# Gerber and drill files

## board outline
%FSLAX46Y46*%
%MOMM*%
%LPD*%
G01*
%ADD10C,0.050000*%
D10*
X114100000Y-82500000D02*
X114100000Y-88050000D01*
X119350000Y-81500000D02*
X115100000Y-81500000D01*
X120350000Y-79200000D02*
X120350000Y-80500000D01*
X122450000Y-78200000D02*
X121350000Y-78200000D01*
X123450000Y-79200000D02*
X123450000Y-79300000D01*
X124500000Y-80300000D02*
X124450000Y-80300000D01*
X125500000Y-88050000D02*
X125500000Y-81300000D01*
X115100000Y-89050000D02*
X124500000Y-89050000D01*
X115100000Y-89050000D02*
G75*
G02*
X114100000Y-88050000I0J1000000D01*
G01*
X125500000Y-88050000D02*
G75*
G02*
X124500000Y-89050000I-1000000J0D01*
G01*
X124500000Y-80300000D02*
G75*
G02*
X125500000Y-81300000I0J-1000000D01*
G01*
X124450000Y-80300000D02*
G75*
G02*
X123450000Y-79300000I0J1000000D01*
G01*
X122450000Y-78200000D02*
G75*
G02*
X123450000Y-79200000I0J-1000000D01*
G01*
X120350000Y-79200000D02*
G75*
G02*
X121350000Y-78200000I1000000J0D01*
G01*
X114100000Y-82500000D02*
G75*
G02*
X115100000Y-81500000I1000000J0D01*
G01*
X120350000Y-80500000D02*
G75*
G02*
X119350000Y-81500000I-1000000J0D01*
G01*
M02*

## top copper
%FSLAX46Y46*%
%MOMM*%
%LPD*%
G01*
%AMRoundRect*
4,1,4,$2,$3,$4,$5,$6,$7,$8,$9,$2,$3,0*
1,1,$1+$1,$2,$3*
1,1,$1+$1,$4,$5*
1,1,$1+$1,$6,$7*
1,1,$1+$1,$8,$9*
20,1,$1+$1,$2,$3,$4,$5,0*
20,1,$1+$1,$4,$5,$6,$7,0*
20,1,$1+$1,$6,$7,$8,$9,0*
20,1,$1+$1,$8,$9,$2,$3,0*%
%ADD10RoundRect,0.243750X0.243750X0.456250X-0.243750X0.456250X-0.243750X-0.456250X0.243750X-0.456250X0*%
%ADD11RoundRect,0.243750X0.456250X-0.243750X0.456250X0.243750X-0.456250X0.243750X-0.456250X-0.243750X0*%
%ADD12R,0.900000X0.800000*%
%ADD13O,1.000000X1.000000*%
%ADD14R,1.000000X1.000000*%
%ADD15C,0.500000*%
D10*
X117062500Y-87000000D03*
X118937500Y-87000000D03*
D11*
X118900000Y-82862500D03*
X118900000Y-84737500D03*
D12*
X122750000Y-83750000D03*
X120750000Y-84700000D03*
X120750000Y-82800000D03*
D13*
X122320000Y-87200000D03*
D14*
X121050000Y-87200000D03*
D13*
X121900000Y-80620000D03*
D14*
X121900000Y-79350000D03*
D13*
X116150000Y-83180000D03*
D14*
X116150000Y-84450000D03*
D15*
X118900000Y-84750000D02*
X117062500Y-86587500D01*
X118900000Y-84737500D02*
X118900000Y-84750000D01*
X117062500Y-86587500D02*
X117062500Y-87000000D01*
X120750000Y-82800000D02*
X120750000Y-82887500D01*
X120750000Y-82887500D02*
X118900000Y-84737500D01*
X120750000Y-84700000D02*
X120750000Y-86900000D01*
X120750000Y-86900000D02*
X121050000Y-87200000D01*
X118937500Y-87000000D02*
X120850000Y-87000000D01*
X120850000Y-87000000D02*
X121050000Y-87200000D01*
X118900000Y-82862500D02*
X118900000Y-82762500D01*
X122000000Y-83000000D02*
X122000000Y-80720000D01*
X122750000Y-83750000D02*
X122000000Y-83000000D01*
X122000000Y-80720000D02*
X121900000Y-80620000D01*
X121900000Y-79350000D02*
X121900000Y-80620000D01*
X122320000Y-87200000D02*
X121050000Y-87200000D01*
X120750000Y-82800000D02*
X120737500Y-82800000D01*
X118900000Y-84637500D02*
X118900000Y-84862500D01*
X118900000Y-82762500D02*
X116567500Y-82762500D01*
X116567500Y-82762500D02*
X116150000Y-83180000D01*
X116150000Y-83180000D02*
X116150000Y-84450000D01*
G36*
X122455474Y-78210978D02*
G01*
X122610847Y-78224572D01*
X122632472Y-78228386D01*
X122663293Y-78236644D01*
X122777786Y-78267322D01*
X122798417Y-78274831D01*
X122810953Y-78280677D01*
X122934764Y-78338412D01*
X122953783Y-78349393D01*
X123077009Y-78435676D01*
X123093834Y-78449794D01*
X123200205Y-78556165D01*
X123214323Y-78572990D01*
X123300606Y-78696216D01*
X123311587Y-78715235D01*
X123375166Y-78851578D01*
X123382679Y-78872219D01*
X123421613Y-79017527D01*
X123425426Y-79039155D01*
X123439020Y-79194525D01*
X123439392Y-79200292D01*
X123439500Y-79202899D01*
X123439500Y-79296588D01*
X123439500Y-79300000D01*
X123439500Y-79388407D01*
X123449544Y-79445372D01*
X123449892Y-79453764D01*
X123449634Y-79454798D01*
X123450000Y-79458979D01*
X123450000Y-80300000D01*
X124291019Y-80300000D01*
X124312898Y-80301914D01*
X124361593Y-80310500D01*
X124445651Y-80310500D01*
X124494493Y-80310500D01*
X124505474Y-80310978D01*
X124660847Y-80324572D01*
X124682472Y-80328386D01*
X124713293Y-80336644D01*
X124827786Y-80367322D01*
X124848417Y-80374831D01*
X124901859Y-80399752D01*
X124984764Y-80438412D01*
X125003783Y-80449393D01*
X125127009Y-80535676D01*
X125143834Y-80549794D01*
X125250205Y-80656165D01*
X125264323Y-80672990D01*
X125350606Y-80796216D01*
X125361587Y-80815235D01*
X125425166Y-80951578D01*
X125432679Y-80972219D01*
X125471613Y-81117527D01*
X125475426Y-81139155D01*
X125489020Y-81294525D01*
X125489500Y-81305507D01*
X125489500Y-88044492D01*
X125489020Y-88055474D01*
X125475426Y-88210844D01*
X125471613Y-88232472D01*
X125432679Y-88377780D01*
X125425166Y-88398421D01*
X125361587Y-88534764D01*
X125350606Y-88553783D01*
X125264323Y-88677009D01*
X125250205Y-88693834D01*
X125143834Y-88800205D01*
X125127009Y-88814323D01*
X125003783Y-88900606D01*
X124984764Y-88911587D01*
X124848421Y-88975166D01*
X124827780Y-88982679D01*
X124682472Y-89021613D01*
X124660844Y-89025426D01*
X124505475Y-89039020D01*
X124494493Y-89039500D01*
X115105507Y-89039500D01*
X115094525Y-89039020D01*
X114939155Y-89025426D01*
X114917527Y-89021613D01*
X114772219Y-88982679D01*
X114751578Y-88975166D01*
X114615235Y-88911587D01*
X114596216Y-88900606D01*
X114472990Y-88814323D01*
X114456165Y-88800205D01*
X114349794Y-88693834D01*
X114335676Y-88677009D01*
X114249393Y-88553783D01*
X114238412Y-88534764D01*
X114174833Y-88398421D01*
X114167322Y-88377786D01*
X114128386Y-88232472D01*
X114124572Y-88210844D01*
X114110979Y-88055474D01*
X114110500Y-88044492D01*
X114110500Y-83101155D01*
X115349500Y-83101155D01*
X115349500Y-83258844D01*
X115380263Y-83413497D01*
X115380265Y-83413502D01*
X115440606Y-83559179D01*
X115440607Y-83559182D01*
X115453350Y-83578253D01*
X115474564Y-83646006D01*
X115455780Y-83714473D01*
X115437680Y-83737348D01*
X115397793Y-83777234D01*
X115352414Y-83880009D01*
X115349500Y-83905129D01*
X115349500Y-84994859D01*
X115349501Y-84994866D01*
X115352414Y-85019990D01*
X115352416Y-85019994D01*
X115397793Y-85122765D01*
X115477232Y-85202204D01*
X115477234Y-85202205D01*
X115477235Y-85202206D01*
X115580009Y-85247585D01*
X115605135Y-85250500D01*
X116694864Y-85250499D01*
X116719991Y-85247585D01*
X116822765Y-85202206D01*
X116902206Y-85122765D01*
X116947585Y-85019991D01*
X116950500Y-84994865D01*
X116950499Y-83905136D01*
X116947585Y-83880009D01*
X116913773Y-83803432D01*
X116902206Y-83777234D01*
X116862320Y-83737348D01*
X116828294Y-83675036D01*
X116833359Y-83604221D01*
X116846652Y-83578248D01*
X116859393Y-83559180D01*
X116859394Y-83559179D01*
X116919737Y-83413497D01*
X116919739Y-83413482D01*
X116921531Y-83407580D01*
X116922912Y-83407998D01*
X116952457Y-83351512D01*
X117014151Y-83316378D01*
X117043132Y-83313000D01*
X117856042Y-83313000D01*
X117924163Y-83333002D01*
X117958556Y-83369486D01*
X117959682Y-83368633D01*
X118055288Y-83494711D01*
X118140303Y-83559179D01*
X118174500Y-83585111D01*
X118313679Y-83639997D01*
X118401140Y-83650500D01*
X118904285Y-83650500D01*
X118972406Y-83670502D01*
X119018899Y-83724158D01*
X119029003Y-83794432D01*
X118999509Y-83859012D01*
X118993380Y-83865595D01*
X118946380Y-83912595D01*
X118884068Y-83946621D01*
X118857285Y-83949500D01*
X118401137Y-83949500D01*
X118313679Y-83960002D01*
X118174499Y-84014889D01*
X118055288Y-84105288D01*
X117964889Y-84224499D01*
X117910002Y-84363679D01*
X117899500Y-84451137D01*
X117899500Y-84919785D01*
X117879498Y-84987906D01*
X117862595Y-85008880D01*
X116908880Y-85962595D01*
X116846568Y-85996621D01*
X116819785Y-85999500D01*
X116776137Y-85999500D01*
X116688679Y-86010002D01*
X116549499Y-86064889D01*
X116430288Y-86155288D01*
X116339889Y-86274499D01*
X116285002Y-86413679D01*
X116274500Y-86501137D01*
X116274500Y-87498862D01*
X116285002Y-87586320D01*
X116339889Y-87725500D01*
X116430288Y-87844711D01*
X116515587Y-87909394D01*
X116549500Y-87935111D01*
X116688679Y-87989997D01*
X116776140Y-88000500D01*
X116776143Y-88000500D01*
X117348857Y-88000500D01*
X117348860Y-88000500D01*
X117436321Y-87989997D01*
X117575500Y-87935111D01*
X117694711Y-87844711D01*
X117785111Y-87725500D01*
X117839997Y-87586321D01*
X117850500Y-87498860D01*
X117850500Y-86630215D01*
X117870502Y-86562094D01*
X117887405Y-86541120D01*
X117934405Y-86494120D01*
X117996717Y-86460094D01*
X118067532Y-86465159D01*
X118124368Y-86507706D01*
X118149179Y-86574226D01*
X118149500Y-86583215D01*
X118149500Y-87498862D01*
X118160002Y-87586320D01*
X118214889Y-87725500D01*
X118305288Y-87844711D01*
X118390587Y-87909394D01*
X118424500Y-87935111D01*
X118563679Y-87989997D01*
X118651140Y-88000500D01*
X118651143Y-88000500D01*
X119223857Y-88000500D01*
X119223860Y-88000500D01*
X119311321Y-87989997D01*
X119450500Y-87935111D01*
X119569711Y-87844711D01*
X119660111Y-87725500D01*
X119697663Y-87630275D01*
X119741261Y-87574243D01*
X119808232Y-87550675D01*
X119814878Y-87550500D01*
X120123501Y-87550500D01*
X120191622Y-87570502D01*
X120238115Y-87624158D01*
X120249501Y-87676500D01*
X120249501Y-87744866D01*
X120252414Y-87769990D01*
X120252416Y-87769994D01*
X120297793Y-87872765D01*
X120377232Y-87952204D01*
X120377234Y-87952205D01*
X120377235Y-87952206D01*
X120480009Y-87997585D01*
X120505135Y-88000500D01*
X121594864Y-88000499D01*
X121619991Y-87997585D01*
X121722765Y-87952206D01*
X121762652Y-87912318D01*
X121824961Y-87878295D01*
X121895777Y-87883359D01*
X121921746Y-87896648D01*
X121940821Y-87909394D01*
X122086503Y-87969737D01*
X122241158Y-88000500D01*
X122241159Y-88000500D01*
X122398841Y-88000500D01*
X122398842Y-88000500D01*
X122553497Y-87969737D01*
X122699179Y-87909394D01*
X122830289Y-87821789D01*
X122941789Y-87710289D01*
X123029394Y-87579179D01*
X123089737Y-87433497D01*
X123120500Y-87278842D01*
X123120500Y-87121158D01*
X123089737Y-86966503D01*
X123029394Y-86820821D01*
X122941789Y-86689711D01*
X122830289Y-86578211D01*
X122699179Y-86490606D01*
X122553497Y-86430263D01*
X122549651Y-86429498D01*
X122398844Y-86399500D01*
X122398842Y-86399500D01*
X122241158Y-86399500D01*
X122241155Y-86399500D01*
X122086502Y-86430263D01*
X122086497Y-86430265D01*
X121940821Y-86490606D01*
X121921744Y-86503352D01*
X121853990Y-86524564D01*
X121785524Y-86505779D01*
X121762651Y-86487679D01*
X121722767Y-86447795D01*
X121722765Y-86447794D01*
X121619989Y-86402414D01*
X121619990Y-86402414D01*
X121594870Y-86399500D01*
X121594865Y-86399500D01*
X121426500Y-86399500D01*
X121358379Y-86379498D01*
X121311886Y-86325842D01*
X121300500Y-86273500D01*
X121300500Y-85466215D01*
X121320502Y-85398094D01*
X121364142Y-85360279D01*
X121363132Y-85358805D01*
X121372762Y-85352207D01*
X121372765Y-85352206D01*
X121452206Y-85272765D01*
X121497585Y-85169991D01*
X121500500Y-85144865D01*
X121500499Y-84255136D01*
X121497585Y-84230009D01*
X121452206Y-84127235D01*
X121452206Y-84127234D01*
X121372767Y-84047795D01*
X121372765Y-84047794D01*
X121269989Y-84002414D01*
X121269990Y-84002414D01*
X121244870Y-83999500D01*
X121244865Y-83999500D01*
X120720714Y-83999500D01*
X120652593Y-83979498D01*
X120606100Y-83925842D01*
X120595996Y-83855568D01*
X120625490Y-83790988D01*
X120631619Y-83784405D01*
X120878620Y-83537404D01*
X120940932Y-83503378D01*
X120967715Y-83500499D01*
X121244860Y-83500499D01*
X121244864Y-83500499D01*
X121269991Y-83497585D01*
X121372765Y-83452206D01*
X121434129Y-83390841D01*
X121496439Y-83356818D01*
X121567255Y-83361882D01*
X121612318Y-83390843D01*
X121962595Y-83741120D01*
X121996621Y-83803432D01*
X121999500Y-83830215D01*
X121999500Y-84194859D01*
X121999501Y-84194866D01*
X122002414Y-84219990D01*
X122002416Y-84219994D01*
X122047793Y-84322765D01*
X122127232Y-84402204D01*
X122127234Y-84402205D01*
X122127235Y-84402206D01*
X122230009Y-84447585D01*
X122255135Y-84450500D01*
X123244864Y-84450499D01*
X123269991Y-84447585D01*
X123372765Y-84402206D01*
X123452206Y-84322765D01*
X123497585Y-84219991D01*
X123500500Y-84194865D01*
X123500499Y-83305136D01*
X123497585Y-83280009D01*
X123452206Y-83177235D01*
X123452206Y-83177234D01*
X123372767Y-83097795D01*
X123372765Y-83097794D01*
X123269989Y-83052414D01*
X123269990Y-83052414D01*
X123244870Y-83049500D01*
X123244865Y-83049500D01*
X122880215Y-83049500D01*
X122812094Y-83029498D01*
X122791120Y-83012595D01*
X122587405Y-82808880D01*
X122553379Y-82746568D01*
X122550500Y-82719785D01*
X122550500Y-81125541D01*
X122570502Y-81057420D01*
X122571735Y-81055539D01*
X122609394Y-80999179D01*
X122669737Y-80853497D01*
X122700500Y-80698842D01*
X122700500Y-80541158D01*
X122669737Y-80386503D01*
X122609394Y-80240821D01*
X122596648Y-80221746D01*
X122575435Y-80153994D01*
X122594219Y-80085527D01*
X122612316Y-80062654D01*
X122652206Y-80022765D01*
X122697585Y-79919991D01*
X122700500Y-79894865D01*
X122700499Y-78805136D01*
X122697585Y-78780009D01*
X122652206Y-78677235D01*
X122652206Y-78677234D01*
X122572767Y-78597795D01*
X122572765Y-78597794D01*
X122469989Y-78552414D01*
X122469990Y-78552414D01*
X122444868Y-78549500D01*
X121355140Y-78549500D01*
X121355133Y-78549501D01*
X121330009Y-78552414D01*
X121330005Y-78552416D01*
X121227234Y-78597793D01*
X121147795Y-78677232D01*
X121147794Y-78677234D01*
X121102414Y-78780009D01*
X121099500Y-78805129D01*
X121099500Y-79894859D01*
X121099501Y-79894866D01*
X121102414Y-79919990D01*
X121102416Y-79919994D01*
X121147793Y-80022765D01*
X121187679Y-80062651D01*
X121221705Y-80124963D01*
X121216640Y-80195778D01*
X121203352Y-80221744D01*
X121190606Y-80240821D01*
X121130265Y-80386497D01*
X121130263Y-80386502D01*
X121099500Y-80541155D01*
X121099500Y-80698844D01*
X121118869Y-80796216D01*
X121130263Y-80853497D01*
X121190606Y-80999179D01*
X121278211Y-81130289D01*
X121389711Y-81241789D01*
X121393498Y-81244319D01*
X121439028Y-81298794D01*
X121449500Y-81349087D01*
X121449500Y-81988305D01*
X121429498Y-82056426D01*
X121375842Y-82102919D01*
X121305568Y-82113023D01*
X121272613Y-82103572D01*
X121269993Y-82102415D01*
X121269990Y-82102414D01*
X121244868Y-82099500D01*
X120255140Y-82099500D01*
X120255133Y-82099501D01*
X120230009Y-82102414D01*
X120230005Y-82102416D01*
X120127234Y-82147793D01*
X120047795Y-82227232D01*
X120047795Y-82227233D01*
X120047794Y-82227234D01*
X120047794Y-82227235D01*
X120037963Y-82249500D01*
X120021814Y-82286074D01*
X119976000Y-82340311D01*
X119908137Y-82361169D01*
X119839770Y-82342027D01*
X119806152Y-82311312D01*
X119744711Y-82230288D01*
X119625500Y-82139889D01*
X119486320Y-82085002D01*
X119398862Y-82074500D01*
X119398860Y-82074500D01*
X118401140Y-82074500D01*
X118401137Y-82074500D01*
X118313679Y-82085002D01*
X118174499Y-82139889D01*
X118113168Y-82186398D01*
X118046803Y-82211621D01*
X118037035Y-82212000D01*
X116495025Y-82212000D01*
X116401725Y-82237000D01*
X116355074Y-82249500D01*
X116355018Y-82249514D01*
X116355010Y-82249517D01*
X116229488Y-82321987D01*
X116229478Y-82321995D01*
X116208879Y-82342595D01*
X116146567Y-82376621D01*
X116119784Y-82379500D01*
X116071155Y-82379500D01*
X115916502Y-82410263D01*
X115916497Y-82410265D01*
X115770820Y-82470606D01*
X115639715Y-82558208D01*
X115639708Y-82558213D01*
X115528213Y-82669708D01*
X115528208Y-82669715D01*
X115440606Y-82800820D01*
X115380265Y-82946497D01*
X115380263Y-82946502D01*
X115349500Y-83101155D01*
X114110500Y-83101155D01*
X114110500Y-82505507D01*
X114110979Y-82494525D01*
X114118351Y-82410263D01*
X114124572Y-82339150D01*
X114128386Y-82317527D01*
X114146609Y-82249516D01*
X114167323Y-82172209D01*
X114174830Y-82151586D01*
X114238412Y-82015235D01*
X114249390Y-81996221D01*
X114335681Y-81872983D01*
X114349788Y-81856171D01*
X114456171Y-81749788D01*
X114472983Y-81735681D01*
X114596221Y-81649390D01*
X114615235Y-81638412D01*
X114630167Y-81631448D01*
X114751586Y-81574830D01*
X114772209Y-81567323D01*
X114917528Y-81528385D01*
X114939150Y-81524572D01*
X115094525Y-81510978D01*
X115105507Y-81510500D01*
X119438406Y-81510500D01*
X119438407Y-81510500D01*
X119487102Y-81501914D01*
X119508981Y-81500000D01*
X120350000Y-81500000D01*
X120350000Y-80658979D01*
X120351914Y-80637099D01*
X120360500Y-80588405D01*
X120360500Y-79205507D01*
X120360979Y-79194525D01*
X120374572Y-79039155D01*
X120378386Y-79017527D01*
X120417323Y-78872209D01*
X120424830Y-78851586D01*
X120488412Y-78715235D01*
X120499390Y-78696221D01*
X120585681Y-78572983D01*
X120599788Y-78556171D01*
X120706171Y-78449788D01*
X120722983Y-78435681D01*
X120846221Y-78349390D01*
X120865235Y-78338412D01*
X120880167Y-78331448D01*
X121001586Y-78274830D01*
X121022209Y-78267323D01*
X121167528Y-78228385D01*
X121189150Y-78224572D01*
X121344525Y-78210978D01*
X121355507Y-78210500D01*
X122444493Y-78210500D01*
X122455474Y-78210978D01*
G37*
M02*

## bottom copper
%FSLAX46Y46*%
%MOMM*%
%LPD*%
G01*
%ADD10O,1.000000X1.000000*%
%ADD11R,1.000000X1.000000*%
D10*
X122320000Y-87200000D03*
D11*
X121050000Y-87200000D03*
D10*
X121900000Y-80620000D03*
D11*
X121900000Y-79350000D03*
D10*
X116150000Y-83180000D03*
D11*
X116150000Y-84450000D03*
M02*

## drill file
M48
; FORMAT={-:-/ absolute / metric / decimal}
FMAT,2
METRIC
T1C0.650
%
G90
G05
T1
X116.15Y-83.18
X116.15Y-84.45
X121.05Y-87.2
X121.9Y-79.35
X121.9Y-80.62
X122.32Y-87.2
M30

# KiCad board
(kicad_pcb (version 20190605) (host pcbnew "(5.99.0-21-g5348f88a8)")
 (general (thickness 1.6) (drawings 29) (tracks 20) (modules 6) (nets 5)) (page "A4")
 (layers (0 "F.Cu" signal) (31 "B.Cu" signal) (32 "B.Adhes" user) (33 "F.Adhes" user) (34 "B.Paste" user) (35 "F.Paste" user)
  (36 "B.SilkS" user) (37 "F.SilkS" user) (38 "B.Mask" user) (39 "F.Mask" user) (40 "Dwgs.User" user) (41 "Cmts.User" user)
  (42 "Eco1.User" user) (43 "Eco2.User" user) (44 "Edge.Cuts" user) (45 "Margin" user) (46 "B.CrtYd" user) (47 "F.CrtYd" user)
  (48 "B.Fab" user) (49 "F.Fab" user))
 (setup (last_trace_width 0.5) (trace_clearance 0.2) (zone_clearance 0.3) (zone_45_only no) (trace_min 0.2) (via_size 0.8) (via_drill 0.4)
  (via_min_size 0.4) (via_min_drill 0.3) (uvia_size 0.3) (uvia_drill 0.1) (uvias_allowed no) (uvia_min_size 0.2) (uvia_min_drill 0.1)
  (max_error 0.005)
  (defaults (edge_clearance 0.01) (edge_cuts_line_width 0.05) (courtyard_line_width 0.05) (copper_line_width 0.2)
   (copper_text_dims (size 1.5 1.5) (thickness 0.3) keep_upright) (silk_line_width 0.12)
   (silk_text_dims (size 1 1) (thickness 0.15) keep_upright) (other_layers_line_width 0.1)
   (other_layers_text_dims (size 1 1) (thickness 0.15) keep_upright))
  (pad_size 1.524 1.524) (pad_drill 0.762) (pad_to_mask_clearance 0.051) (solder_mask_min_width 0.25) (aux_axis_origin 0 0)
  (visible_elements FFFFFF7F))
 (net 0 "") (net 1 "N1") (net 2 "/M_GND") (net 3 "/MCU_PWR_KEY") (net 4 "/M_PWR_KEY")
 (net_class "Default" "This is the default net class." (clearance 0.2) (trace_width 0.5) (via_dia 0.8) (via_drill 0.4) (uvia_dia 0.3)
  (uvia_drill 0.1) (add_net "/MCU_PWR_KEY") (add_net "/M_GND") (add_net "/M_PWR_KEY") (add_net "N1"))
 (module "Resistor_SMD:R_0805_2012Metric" (layer "F.Cu") (at 118 87 180)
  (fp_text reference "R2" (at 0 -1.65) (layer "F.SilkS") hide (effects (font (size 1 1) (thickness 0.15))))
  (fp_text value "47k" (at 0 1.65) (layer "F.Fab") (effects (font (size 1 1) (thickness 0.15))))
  (pad "2" smd roundrect (at 0.9375 0 180) (size 0.975 1.4) (layers "F.Cu" "F.Paste" "F.Mask") (roundrect_rratio 0.25) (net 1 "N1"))
  (pad "1" smd roundrect (at -0.9375 0 180) (size 0.975 1.4) (layers "F.Cu" "F.Paste" "F.Mask") (roundrect_rratio 0.25) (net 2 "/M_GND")))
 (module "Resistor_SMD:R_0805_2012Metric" (layer "F.Cu") (at 118.9 83.8 90)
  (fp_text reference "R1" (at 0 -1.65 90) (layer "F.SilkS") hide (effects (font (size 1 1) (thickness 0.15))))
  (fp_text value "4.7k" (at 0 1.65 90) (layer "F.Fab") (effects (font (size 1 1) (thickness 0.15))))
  (pad "2" smd roundrect (at 0.9375 0 90) (size 0.975 1.4) (layers "F.Cu" "F.Paste" "F.Mask") (roundrect_rratio 0.25) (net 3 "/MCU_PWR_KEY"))
  (pad "1" smd roundrect (at -0.9375 0 90) (size 0.975 1.4) (layers "F.Cu" "F.Paste" "F.Mask") (roundrect_rratio 0.25) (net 1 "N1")))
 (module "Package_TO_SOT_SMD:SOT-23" (layer "F.Cu") (at 121.75 83.75)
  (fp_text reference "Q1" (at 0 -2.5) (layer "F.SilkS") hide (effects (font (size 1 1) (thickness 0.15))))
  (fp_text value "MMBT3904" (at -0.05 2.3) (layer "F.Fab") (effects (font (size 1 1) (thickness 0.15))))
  (pad "3" smd rect (at 1 0) (size 0.9 0.8) (layers "F.Cu" "F.Paste" "F.Mask") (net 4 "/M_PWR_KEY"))
  (pad "2" smd rect (at -1 0.95) (size 0.9 0.8) (layers "F.Cu" "F.Paste" "F.Mask") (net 2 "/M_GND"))
  (pad "1" smd rect (at -1 -0.95) (size 0.9 0.8) (layers "F.Cu" "F.Paste" "F.Mask") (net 1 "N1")))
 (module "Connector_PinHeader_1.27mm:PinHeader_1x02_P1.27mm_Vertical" (layer "F.Cu") (at 121.05 87.2 90)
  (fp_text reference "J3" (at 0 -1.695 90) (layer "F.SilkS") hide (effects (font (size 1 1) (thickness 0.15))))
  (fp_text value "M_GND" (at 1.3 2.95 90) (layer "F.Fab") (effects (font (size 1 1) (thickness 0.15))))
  (pad "2" thru_hole oval (at 0 1.27 90) (size 1 1) (drill 0.65) (layers *.Cu *.Mask) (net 2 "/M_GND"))
  (pad "1" thru_hole rect (at 0 0 90) (size 1 1) (drill 0.65) (layers *.Cu *.Mask) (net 2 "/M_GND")))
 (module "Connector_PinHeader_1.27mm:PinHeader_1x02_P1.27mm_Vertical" (layer "F.Cu") (at 121.9 79.35)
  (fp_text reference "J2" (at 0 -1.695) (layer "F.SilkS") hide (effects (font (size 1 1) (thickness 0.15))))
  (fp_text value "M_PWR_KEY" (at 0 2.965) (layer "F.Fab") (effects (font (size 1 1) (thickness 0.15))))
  (pad "2" thru_hole oval (at 0 1.27) (size 1 1) (drill 0.65) (layers *.Cu *.Mask) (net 4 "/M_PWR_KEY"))
  (pad "1" thru_hole rect (at 0 0) (size 1 1) (drill 0.65) (layers *.Cu *.Mask) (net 4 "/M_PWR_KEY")))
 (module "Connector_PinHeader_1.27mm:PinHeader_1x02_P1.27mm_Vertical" (layer "F.Cu") (at 116.15 84.45 180)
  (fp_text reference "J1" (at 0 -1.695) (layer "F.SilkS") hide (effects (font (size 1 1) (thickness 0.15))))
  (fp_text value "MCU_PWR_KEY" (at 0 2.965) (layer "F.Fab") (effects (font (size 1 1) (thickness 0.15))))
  (pad "2" thru_hole oval (at 0 1.27 180) (size 1 1) (drill 0.65) (layers *.Cu *.Mask) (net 3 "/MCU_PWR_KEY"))
  (pad "1" thru_hole rect (at 0 0 180) (size 1 1) (drill 0.65) (layers *.Cu *.Mask) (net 3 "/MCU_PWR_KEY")))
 (gr_line (start 114.1 82.5) (end 114.1 88.05) (layer "Edge.Cuts") (width 0.05))
 (gr_line (start 119.35 81.5) (end 115.1 81.5) (layer "Edge.Cuts") (width 0.05))
 (gr_line (start 120.35 79.2) (end 120.35 80.5) (layer "Edge.Cuts") (width 0.05))
 (gr_line (start 122.45 78.2) (end 121.35 78.2) (layer "Edge.Cuts") (width 0.05))
 (gr_line (start 123.45 79.2) (end 123.45 79.3) (layer "Edge.Cuts") (width 0.05))
 (gr_line (start 124.5 80.3) (end 124.45 80.3) (layer "Edge.Cuts") (width 0.05))
 (gr_line (start 125.5 88.05) (end 125.5 81.3) (layer "Edge.Cuts") (width 0.05))
 (gr_line (start 115.1 89.05) (end 124.5 89.05) (layer "Edge.Cuts") (width 0.05))
 (gr_arc (start 115.1 88.05) (end 114.1 88.05) (angle -90) (layer "Edge.Cuts") (width 0.05))
 (gr_arc (start 124.5 88.05) (end 124.5 89.05) (angle -90) (layer "Edge.Cuts") (width 0.05))
 (gr_arc (start 124.5 81.3) (end 125.5 81.3) (angle -90) (layer "Edge.Cuts") (width 0.05))
 (gr_arc (start 124.45 79.3) (end 123.45 79.3) (angle -90) (layer "Edge.Cuts") (width 0.05))
 (gr_arc (start 122.45 79.2) (end 123.45 79.2) (angle -90) (layer "Edge.Cuts") (width 0.05))
 (gr_arc (start 121.35 79.2) (end 121.35 78.2) (angle -90) (layer "Edge.Cuts") (width 0.05))
 (gr_arc (start 115.1 82.5) (end 115.1 81.5) (angle -90) (layer "Edge.Cuts") (width 0.05))
 (gr_arc (start 119.35 80.5) (end 119.35 81.5) (angle -90) (layer "Edge.Cuts") (width 0.05))
 (segment (start 118.9 84.75) (end 117.0625 86.5875) (width 0.5) (layer "F.Cu") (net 1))
 (segment (start 118.9 84.7375) (end 118.9 84.75) (width 0.5) (layer "F.Cu") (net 1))
 (segment (start 117.0625 86.5875) (end 117.0625 87) (width 0.5) (layer "F.Cu") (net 1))
 (segment (start 120.75 82.8) (end 120.75 82.8875) (width 0.5) (layer "F.Cu") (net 1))
 (segment (start 120.75 82.8875) (end 118.9 84.7375) (width 0.5) (layer "F.Cu") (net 1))
 (segment (start 120.75 84.7) (end 120.75 86.9) (width 0.5) (layer "F.Cu") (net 2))
 (segment (start 120.75 86.9) (end 121.05 87.2) (width 0.5) (layer "F.Cu") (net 2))
 (segment (start 118.9375 87) (end 120.85 87) (width 0.5) (layer "F.Cu") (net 2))
 (segment (start 120.85 87) (end 121.05 87.2) (width 0.5) (layer "F.Cu") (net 2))
 (segment (start 118.9 82.8625) (end 118.9 82.7625) (width 0.5) (layer "F.Cu") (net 3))
 (segment (start 122 83) (end 122 80.72) (width 0.5) (layer "F.Cu") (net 4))
 (segment (start 122.75 83.75) (end 122 83) (width 0.5) (layer "F.Cu") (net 4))
 (segment (start 122 80.72) (end 121.9 80.62) (width 0.5) (layer "F.Cu") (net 4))
 (segment (start 121.9 79.35) (end 121.9 80.62) (width 0.5) (layer "F.Cu") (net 4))
 (segment (start 122.32 87.2) (end 121.05 87.2) (width 0.5) (layer "F.Cu") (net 2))
 (segment (start 120.75 82.8) (end 120.7375 82.8) (width 0.5) (layer "F.Cu") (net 1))
 (segment (start 118.9 84.6375) (end 118.9 84.8625) (width 0.5) (layer "F.Cu") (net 1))
 (segment (start 118.9 82.7625) (end 116.5675 82.7625) (width 0.5) (layer "F.Cu") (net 3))
 (segment (start 116.5675 82.7625) (end 116.15 83.18) (width 0.5) (layer "F.Cu") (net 3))
 (segment (start 116.15 83.18) (end 116.15 84.45) (width 0.5) (layer "F.Cu") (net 3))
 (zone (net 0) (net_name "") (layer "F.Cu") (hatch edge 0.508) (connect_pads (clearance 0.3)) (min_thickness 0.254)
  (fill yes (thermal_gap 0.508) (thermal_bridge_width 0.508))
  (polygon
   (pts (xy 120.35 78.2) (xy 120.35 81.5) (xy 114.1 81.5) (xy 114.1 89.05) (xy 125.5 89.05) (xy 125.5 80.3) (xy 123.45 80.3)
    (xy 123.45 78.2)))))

